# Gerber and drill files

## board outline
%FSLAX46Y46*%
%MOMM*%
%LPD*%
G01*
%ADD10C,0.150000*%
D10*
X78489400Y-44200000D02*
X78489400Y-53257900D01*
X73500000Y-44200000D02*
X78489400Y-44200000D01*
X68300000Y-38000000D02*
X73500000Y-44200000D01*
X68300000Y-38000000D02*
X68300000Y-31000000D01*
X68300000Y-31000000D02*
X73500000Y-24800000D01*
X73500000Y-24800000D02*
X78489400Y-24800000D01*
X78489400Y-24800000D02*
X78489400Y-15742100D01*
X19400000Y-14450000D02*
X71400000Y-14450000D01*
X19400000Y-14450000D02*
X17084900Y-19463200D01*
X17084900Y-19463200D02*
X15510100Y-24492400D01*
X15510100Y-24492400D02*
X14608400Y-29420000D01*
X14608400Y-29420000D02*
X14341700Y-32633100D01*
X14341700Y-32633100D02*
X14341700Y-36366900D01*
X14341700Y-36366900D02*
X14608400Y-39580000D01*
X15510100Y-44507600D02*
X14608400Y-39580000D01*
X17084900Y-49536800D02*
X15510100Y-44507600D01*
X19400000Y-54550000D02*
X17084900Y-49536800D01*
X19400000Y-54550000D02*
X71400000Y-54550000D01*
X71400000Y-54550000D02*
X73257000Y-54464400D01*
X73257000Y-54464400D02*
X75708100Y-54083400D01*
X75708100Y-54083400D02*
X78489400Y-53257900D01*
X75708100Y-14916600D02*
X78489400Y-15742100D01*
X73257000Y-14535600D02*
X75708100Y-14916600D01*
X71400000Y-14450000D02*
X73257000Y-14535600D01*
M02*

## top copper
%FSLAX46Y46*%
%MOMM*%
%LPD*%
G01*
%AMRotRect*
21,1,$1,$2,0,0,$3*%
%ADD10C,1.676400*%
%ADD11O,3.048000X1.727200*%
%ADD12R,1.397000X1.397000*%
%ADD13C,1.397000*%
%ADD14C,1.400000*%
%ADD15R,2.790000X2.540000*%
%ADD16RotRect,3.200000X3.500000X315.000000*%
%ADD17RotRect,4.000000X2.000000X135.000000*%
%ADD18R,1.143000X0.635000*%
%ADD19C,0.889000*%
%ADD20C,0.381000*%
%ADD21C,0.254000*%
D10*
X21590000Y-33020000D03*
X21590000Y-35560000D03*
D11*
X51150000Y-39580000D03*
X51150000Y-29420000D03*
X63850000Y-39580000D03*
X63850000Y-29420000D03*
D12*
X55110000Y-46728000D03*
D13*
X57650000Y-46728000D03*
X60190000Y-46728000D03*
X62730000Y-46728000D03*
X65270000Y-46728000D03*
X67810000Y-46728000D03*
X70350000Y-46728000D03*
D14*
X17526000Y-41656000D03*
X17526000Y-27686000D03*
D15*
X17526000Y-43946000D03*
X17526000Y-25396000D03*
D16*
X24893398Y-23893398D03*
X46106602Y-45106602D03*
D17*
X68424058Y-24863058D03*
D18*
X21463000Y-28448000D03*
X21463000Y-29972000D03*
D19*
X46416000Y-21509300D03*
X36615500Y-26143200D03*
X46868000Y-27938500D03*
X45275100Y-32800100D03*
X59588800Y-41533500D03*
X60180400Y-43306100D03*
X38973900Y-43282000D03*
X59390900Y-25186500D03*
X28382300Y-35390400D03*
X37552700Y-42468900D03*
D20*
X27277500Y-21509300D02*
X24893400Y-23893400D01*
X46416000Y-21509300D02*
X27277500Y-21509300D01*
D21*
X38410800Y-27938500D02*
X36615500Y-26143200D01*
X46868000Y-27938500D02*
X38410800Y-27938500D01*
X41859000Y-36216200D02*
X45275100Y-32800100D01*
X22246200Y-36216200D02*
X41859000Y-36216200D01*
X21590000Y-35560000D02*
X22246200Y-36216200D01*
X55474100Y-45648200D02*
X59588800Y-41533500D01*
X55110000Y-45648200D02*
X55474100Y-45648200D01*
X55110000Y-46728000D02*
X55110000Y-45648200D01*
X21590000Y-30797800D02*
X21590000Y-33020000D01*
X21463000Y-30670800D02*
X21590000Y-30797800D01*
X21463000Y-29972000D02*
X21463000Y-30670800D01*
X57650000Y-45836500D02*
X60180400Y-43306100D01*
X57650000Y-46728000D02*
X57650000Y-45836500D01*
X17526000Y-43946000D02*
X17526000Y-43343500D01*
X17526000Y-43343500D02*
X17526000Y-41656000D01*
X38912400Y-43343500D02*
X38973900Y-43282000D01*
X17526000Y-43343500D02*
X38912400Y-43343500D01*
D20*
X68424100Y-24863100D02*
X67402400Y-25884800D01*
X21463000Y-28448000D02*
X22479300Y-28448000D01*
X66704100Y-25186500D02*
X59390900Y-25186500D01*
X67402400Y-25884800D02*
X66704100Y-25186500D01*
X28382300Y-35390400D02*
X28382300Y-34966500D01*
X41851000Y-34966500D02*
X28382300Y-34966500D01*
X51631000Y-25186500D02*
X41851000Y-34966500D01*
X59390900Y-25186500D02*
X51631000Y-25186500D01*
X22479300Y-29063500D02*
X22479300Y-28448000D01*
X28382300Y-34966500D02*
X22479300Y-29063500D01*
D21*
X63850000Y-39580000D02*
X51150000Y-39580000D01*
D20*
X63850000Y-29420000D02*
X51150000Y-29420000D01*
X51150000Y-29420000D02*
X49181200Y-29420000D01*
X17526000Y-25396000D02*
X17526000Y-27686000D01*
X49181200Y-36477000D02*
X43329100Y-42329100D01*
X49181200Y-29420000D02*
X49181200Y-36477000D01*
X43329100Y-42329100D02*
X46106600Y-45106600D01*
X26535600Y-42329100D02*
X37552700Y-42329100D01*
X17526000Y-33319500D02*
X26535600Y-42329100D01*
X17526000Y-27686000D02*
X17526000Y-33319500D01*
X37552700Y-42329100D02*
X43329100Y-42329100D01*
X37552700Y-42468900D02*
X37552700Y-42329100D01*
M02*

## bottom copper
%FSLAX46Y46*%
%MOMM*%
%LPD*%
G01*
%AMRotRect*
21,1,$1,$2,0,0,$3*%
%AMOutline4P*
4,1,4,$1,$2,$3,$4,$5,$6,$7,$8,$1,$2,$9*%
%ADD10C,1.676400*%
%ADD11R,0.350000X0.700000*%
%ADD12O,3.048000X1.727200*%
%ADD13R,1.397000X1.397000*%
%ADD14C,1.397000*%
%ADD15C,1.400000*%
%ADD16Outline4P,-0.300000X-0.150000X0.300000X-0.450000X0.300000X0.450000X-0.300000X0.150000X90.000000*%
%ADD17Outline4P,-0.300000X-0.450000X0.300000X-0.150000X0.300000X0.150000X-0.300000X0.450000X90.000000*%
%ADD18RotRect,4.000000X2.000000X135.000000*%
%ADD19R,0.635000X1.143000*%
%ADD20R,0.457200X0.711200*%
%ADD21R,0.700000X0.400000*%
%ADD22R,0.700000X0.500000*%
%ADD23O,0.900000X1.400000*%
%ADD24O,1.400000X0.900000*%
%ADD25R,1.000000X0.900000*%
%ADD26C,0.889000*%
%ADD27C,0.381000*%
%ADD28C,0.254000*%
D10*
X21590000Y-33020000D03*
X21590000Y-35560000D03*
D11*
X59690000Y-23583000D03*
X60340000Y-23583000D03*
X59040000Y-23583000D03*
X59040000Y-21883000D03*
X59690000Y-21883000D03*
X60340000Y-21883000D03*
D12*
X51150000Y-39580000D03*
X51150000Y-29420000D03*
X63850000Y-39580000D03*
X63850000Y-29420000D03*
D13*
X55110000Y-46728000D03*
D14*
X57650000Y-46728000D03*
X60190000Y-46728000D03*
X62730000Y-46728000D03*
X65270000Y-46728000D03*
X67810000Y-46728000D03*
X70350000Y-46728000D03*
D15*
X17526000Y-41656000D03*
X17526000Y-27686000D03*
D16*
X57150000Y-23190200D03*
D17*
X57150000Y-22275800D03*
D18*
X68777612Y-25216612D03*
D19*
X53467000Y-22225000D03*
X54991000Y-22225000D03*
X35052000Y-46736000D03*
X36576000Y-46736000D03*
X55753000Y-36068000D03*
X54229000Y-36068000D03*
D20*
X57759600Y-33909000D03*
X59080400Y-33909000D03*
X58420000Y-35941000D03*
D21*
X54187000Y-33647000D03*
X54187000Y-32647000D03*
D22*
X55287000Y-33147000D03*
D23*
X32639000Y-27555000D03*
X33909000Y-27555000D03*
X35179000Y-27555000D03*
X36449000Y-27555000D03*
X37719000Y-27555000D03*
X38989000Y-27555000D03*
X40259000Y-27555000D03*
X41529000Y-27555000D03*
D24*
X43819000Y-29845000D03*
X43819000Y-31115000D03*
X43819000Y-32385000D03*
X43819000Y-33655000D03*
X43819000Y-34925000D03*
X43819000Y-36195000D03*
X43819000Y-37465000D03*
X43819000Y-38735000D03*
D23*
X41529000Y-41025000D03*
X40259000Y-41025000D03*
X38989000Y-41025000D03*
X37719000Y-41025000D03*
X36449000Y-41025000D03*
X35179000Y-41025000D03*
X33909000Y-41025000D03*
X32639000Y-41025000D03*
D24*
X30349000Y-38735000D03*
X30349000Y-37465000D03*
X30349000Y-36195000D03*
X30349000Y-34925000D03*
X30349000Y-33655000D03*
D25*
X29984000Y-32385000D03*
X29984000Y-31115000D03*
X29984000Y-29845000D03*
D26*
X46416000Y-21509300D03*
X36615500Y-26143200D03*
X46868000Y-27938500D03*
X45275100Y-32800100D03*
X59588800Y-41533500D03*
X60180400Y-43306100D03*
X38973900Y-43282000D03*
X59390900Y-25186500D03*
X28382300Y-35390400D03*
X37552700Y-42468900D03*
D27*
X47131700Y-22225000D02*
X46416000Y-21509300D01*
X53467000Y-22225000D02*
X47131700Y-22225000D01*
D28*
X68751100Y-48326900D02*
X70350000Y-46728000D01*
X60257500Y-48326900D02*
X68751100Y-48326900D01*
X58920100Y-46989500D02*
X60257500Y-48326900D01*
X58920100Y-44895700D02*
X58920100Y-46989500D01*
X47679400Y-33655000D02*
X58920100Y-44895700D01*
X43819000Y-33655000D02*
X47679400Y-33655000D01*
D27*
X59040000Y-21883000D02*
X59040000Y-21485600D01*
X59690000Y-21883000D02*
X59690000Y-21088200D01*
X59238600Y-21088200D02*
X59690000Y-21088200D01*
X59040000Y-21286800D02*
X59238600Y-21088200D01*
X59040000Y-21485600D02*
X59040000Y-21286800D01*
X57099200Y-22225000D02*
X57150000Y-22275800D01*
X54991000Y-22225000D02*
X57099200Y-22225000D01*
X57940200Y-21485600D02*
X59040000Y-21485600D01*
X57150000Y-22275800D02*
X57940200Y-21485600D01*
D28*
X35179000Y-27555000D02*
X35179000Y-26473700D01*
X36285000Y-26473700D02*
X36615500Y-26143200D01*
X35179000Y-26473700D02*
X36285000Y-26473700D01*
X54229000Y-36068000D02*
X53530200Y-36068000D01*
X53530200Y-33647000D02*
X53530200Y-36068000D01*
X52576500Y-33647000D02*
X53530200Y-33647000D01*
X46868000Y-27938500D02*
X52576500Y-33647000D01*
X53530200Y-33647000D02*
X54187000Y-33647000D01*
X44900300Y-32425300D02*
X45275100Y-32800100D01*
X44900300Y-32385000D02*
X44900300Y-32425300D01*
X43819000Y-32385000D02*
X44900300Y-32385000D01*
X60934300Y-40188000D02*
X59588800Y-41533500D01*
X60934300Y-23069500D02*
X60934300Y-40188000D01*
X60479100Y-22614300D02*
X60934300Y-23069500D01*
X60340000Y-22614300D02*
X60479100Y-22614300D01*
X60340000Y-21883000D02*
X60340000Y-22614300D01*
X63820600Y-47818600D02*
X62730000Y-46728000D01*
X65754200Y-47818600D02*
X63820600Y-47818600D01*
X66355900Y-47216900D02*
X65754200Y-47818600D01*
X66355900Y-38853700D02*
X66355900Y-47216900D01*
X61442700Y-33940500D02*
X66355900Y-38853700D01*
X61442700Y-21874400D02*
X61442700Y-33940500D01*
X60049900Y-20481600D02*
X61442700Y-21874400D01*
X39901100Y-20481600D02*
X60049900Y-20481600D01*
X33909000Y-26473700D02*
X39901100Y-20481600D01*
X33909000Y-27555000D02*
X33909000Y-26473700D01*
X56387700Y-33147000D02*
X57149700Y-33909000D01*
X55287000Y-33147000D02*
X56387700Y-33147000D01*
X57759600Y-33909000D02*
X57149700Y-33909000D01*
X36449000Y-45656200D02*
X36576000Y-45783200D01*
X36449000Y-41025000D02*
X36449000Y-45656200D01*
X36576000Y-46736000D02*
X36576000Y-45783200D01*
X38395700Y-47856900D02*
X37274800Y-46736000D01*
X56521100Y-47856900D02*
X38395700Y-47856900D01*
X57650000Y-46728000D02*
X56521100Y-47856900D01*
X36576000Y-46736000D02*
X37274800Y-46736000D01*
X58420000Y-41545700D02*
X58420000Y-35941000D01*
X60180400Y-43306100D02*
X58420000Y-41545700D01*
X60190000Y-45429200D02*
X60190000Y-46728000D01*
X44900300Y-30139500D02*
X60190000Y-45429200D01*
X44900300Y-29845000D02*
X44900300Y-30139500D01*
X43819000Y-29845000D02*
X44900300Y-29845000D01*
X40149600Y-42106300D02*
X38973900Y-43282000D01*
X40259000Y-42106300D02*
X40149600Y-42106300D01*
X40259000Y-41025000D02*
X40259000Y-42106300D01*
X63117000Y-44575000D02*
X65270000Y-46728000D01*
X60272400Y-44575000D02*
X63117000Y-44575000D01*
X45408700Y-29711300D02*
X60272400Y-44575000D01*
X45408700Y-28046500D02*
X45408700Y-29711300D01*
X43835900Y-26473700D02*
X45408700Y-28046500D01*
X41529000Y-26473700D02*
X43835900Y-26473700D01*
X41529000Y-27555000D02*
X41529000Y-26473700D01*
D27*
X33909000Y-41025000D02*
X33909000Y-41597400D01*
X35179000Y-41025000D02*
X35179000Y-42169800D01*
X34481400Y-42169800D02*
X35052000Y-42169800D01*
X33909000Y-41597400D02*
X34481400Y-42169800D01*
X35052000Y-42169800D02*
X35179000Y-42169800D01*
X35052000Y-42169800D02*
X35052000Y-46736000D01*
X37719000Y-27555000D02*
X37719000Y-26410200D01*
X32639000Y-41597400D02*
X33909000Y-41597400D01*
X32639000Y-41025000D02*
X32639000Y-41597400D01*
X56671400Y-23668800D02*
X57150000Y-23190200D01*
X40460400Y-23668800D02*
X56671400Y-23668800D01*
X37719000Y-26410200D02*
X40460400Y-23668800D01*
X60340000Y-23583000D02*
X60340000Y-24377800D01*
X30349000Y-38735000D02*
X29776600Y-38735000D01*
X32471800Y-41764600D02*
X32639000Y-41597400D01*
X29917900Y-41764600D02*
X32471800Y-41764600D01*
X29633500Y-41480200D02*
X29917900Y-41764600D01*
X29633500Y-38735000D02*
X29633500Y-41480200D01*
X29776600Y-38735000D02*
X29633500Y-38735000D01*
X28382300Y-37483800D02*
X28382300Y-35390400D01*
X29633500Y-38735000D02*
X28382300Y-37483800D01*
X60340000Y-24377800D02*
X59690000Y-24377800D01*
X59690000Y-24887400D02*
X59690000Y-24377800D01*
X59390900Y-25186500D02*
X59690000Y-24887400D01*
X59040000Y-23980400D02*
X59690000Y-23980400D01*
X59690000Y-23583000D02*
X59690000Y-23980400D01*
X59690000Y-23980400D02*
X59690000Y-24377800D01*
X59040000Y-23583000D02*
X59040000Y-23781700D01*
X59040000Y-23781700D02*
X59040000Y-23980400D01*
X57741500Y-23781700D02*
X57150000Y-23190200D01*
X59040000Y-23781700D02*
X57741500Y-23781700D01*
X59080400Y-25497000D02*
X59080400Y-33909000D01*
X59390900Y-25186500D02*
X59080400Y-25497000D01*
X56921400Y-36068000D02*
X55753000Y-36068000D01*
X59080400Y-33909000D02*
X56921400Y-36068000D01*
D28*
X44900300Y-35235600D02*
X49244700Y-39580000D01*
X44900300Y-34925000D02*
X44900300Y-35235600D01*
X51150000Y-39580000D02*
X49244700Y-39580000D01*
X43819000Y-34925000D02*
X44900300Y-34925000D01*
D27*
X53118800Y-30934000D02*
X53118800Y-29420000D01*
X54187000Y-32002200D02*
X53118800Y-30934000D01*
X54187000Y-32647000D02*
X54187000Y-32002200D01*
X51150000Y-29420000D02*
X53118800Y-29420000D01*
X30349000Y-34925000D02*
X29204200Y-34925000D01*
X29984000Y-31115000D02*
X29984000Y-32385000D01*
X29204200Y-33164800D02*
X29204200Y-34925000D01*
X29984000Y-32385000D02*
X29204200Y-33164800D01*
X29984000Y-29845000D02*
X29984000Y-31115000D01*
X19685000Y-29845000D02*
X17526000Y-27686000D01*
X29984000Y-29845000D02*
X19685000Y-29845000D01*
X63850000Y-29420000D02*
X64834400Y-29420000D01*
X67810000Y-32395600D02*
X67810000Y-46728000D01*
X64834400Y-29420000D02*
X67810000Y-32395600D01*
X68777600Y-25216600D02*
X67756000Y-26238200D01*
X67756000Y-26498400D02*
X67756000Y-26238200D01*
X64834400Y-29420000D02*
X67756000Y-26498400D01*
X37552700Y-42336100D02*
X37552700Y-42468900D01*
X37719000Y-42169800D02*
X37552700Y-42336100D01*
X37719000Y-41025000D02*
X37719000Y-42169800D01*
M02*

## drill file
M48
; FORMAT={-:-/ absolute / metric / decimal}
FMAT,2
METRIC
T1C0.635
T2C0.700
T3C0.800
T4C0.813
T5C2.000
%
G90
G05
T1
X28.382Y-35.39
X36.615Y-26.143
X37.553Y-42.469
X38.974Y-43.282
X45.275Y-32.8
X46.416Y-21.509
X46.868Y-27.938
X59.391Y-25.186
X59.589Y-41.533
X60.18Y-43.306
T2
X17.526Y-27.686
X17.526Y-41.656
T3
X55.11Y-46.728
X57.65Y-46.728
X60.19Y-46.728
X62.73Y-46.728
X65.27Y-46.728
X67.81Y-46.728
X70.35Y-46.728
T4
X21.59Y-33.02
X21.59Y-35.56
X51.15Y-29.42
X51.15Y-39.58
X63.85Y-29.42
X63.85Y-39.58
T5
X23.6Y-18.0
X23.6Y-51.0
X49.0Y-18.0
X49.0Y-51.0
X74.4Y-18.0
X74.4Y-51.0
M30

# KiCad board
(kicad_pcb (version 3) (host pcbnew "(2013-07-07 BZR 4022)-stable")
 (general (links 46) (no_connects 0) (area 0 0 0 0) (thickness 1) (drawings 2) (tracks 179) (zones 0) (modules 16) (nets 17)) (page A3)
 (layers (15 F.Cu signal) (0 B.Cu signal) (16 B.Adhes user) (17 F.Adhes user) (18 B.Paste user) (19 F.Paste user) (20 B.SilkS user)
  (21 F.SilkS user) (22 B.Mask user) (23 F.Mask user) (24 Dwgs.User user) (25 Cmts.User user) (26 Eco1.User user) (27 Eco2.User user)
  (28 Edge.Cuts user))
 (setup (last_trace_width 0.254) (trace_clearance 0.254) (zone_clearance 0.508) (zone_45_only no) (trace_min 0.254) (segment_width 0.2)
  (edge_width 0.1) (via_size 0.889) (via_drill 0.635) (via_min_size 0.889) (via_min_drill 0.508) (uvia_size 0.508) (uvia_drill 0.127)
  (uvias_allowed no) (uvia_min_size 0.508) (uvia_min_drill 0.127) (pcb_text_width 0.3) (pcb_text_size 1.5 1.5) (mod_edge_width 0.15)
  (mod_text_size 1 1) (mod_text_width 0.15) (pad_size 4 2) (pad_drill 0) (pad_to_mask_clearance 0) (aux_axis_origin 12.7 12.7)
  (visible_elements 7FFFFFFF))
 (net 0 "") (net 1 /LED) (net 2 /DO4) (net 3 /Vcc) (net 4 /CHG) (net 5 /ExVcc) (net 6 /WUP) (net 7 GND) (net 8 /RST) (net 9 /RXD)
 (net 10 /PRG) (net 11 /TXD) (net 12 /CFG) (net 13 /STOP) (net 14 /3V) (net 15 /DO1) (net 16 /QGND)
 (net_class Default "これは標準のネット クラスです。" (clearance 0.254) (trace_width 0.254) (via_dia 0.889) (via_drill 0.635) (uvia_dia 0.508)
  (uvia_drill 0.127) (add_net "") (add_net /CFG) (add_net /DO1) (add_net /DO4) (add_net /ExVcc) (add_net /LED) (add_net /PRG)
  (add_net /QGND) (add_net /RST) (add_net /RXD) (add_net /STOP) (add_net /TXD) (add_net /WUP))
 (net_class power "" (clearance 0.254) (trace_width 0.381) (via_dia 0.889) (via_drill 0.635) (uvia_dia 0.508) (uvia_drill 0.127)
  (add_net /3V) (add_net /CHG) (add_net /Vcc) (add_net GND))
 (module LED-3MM (layer F.Cu) (at 21.59 34.29 270)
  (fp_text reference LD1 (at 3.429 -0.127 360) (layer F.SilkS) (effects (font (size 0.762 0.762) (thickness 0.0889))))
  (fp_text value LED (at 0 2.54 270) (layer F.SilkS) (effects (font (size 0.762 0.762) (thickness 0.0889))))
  (pad 1 thru_hole circle (at -1.27 0 270) (size 1.6764 1.6764) (drill 0.8128) (layers *.Cu *.Mask F.SilkS) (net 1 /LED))
  (pad 2 thru_hole circle (at 1.27 0 270) (size 1.6764 1.6764) (drill 0.8128) (layers *.Cu *.Mask F.SilkS) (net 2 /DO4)))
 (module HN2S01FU (layer B.Cu) (at 59.69 22.733 90)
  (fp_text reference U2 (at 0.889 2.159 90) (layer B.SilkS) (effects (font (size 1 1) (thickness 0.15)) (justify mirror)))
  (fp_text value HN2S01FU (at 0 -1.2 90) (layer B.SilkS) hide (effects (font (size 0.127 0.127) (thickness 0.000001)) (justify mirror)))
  (pad 2 smd rect (at -0.85 0 90) (size 0.7 0.35) (layers B.Cu B.Paste B.Mask) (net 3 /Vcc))
  (pad 1 smd rect (at -0.85 0.65 90) (size 0.7 0.35) (layers B.Cu B.Paste B.Mask) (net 3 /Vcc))
  (pad 3 smd rect (at -0.85 -0.65 90) (size 0.7 0.35) (layers B.Cu B.Paste B.Mask) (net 3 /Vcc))
  (pad 4 smd rect (at 0.85 -0.65 90) (size 0.7 0.35) (layers B.Cu B.Paste B.Mask) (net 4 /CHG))
  (pad 5 smd rect (at 0.85 0 90) (size 0.7 0.35) (layers B.Cu B.Paste B.Mask) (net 4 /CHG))
  (pad 6 smd rect (at 0.85 0.65 90) (size 0.7 0.35) (layers B.Cu B.Paste B.Mask) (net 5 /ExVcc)))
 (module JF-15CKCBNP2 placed (layer F.Cu) (at 57.5 34.5 180)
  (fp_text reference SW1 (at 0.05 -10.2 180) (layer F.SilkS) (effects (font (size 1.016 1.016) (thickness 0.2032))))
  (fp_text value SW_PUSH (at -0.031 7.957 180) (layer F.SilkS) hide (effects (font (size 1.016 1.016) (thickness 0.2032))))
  (pad 1 thru_hole oval (at 6.35 -5.08 180) (size 3.048 1.7272) (drill 0.8128) (layers *.Cu *.Mask F.SilkS) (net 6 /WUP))
  (pad 2 thru_hole oval (at 6.35 5.08 180) (size 3.048 1.7272) (drill 0.8128) (layers *.Cu *.Mask F.SilkS) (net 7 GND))
  (pad 1 thru_hole oval (at -6.35 -5.08 180) (size 3.048 1.7272) (drill 0.8128) (layers *.Cu *.Mask F.SilkS) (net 6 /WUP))
  (pad 2 thru_hole oval (at -6.35 5.08 180) (size 3.048 1.7272) (drill 0.8128) (layers *.Cu *.Mask F.SilkS) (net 7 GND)))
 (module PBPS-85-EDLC (layer F.Cu) (at 49 34.5)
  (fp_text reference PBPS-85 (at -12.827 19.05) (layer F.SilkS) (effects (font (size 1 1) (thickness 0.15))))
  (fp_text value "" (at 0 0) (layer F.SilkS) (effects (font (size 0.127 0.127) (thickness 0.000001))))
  (fp_line (start 29.4894 9.7) (end 29.4894 18.7579) (layer Edge.Cuts) (width 0.15))
  (fp_line (start 24.5 9.7) (end 29.4894 9.7) (layer Edge.Cuts) (width 0.15))
  (fp_line (start 19.3 3.5) (end 24.5 9.7) (layer Edge.Cuts) (width 0.15))
  (fp_line (start 19.3 3.5) (end 19.3 -3.5) (layer Edge.Cuts) (width 0.15))
  (fp_line (start 19.3 -3.5) (end 24.5 -9.7) (layer Edge.Cuts) (width 0.15))
  (fp_line (start 24.5 -9.7) (end 29.4894 -9.7) (layer Edge.Cuts) (width 0.15))
  (fp_line (start 29.4894 -9.7) (end 29.4894 -18.7579) (layer Edge.Cuts) (width 0.15))
  (fp_line (start -29.6 -20.05) (end 22.4 -20.05) (layer Edge.Cuts) (width 0.15))
  (fp_line (start -29.6 -20.05) (end -31.9151 -15.0368) (layer Edge.Cuts) (width 0.15))
  (fp_line (start -31.9151 -15.0368) (end -33.4899 -10.0076) (layer Edge.Cuts) (width 0.15))
  (fp_line (start -33.4899 -10.0076) (end -34.3916 -5.08) (layer Edge.Cuts) (width 0.15))
  (fp_line (start -34.3916 -5.08) (end -34.6583 -1.8669) (layer Edge.Cuts) (width 0.15))
  (fp_line (start -34.6583 -1.8669) (end -34.6583 1.8669) (layer Edge.Cuts) (width 0.15))
  (fp_line (start -34.6583 1.8669) (end -34.3916 5.08) (layer Edge.Cuts) (width 0.15))
  (fp_line (start -33.4899 10.0076) (end -34.3916 5.08) (layer Edge.Cuts) (width 0.15))
  (fp_line (start -31.9151 15.0368) (end -33.4899 10.0076) (layer Edge.Cuts) (width 0.15))
  (fp_line (start -29.6 20.05) (end -31.9151 15.0368) (layer Edge.Cuts) (width 0.15))
  (fp_line (start -29.6 20.05) (end 22.4 20.05) (layer Edge.Cuts) (width 0.15))
  (fp_line (start 22.4 20.05) (end 24.257 19.9644) (layer Edge.Cuts) (width 0.15))
  (fp_line (start 24.257 19.9644) (end 26.7081 19.5834) (layer Edge.Cuts) (width 0.15))
  (fp_line (start 26.7081 19.5834) (end 29.4894 18.7579) (layer Edge.Cuts) (width 0.15))
  (fp_line (start 26.7081 -19.5834) (end 29.4894 -18.7579) (layer Edge.Cuts) (width 0.15))
  (fp_line (start 24.257 -19.9644) (end 26.7081 -19.5834) (layer Edge.Cuts) (width 0.15))
  (fp_line (start 22.4 -20.05) (end 24.257 -19.9644) (layer Edge.Cuts) (width 0.15))
  (pad "" np_thru_hole circle (at 0 -16.5) (size 2 2) (drill 2) (layers *.Cu *.Mask F.SilkS) (clearance 1))
  (pad "" np_thru_hole circle (at 0 16.5) (size 2 2) (drill 2) (layers *.Cu *.Mask F.SilkS) (clearance 1))
  (pad "" np_thru_hole circle (at -25.4 -16.5) (size 2 2) (drill 2) (layers *.Cu *.Mask F.SilkS) (clearance 1))
  (pad "" np_thru_hole circle (at -25.4 16.5) (size 2 2) (drill 2) (layers *.Cu *.Mask F.SilkS) (clearance 1))
  (pad "" np_thru_hole circle (at 25.4 -16.5) (size 2 2) (drill 2) (layers *.Cu *.Mask F.SilkS) (clearance 1))
  (pad "" np_thru_hole circle (at 25.4 16.5) (size 2 2) (drill 2) (layers *.Cu *.Mask F.SilkS) (clearance 1)))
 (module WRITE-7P (layer F.Cu) (at 62.73 46.728)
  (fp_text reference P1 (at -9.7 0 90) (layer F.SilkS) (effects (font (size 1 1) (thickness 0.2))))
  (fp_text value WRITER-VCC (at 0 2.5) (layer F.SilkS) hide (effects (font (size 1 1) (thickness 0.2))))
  (pad 0 thru_hole rect (at -7.62 0) (size 1.397 1.397) (drill 0.8) (layers *.Cu *.Mask F.SilkS) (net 5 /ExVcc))
  (pad 1 thru_hole circle (at -5.08 0) (size 1.397 1.397) (drill 0.8) (layers *.Cu *.SilkS *.Mask) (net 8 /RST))
  (pad 2 thru_hole circle (at -2.54 0) (size 1.397 1.397) (drill 0.8) (layers *.Cu *.SilkS *.Mask) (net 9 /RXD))
  (pad 3 thru_hole circle (at 0 0) (size 1.397 1.397) (drill 0.8) (layers *.Cu *.SilkS *.Mask) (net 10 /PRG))
  (pad 4 thru_hole circle (at 2.54 0) (size 1.397 1.397) (drill 0.8) (layers *.Cu *.SilkS *.Mask) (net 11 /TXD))
  (pad 5 thru_hole circle (at 5.08 0) (size 1.397 1.397) (drill 0.8) (layers *.Cu *.SilkS *.Mask) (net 7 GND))
  (pad 6 thru_hole circle (at 7.62 0) (size 1.397 1.397) (drill 0.8) (layers *.Cu *.SilkS *.Mask) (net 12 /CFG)))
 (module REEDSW (layer F.Cu) (at 17.526 34.671 90)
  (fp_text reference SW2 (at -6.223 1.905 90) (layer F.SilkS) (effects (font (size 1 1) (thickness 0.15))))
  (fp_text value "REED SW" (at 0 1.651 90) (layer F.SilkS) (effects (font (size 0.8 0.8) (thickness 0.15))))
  (pad 1 thru_hole circle (at -6.985 0 90) (size 1.4 1.4) (drill 0.7) (layers *.Cu *.Mask F.SilkS) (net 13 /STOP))
  (pad 2 thru_hole circle (at 6.985 0 90) (size 1.4 1.4) (drill 0.7) (layers *.Cu *.Mask F.SilkS) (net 7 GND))
  (pad 1 smd rect (at -9.275 0 90) (size 2.54 2.79) (layers F.Cu F.Paste F.Mask) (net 13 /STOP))
  (pad 2 smd rect (at 9.275 0 90) (size 2.54 2.79) (layers F.Cu F.Paste F.Mask) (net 7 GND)))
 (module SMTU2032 (layer F.Cu) (at 35.5 34.5 315)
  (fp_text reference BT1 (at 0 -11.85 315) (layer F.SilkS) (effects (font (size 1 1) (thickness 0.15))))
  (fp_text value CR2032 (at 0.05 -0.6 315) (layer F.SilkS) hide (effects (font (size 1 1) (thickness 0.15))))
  (pad 1 smd rect (at -15 0 315) (size 3.2 3.5) (layers F.Cu F.Paste F.Mask) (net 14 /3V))
  (pad 2 smd rect (at 15 0 315) (size 3.2 3.5) (layers F.Cu F.Paste F.Mask) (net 7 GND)))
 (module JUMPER (layer B.Cu) (at 57.15 22.733 90)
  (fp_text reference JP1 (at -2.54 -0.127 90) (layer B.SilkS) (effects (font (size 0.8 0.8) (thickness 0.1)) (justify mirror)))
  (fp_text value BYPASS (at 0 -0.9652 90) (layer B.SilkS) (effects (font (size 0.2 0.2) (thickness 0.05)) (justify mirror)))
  (pad 1 smd trapezoid (at -0.4572 0 90) (size 0.6 0.6) (rect_delta -0.3 0) (layers B.Cu B.Paste B.Mask) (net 3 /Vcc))
  (pad 2 smd trapezoid (at 0.4572 0 90) (size 0.6 0.6) (rect_delta 0.3 0) (layers B.Cu B.Paste B.Mask) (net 4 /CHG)))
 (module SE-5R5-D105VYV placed (layer F.Cu) (at 77.97 34.409 135)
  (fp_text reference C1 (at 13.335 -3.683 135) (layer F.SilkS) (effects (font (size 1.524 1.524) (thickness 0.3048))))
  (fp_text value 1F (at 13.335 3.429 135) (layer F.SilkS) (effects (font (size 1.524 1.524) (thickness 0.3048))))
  (pad 1 smd rect (at 13.5 0 135) (size 4 2) (layers F.Cu F.Paste F.Mask) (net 3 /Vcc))
  (pad 2 smd rect (at 13 0 135) (size 4 2) (layers B.Cu B.Paste B.Mask) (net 7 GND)))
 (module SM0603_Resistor (layer F.Cu) (at 21.463 29.21 270)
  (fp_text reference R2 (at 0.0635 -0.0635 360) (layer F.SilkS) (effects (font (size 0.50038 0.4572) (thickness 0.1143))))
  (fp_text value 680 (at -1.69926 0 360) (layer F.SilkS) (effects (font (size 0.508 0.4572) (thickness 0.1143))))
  (pad 1 smd rect (at -0.762 0 270) (size 0.635 1.143) (layers F.Cu F.Paste F.Mask) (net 3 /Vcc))
  (pad 2 smd rect (at 0.762 0 270) (size 0.635 1.143) (layers F.Cu F.Paste F.Mask) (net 1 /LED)))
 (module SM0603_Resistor (layer B.Cu) (at 54.229 22.225)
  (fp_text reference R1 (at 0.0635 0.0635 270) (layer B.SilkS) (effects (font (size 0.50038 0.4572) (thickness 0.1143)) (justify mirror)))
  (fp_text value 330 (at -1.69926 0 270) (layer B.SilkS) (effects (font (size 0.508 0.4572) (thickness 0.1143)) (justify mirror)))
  (pad 1 smd rect (at -0.762 0) (size 0.635 1.143) (layers B.Cu B.Paste B.Mask) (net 14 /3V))
  (pad 2 smd rect (at 0.762 0) (size 0.635 1.143) (layers B.Cu B.Paste B.Mask) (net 4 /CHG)))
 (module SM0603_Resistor (layer B.Cu) (at 35.814 46.736)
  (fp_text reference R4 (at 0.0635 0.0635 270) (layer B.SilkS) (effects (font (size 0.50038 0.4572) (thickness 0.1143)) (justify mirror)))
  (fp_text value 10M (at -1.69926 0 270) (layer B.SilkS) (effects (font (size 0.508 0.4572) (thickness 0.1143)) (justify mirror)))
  (pad 1 smd rect (at -0.762 0) (size 0.635 1.143) (layers B.Cu B.Paste B.Mask) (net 3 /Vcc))
  (pad 2 smd rect (at 0.762 0) (size 0.635 1.143) (layers B.Cu B.Paste B.Mask) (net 8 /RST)))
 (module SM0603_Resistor (layer B.Cu) (at 54.991 36.068 180)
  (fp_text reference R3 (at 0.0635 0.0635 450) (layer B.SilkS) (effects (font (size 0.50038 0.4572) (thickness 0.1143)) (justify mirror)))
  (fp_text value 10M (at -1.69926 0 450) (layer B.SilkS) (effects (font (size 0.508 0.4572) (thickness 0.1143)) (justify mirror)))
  (pad 1 smd rect (at -0.762 0 180) (size 0.635 1.143) (layers B.Cu B.Paste B.Mask) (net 3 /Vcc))
  (pad 2 smd rect (at 0.762 0 180) (size 0.635 1.143) (layers B.Cu B.Paste B.Mask) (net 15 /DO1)))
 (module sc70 (layer B.Cu) (at 58.42 34.925)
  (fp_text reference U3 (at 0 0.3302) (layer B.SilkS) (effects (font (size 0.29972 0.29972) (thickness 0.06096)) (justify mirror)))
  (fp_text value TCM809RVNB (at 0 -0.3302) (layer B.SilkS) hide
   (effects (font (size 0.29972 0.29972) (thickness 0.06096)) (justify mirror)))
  (pad 1 smd rect (at -0.6604 -1.016) (size 0.4572 0.7112) (layers B.Cu B.Paste B.Mask) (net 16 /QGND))
  (pad 3 smd rect (at 0.6604 -1.016) (size 0.4572 0.7112) (layers B.Cu B.Paste B.Mask) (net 3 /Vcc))
  (pad 2 smd rect (at 0 1.016) (size 0.4572 0.7112) (layers B.Cu B.Paste B.Mask) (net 8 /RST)))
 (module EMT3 (layer B.Cu) (at 54.737 33.147 90)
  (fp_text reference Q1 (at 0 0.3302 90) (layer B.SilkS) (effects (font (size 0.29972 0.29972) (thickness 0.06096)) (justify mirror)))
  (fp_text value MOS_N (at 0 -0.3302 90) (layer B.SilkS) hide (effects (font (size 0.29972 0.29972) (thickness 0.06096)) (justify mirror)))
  (pad G smd rect (at -0.5 -0.55 90) (size 0.4 0.7) (layers B.Cu B.Paste B.Mask) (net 15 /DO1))
  (pad S smd rect (at 0.5 -0.55 90) (size 0.4 0.7) (layers B.Cu B.Paste B.Mask) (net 7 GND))
  (pad D smd rect (at 0 0.55 90) (size 0.5 0.7) (layers B.Cu B.Paste B.Mask) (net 16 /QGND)))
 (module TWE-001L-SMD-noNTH (layer B.Cu) (at 37.084 34.29 270)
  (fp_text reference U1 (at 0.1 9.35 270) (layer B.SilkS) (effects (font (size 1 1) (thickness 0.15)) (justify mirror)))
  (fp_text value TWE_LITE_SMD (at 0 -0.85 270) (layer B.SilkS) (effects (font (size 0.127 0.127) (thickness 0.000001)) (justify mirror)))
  (pad 1 smd oval (at -6.735 4.445 180) (size 0.9 1.4) (layers B.Cu B.Paste B.Mask))
  (pad 2 smd oval (at -6.735 3.175 180) (size 0.9 1.4) (layers B.Cu B.Paste B.Mask) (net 10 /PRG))
  (pad 3 smd oval (at -6.735 1.905 180) (size 0.9 1.4) (layers B.Cu B.Paste B.Mask) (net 15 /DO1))
  (pad 4 smd oval (at -6.735 0.635 180) (size 0.9 1.4) (layers B.Cu B.Paste B.Mask))
  (pad 5 smd oval (at -6.735 -0.635 180) (size 0.9 1.4) (layers B.Cu B.Paste B.Mask) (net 3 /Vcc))
  (pad 6 smd oval (at -6.735 -1.905 180) (size 0.9 1.4) (layers B.Cu B.Paste B.Mask))
  (pad 7 smd oval (at -6.735 -3.175 180) (size 0.9 1.4) (layers B.Cu B.Paste B.Mask))
  (pad 8 smd oval (at -6.735 -4.445 180) (size 0.9 1.4) (layers B.Cu B.Paste B.Mask) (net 11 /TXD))
  (pad 9 smd oval (at -4.445 -6.735 270) (size 0.9 1.4) (layers B.Cu B.Paste B.Mask) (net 9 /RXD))
  (pad 10 smd oval (at -3.175 -6.735 270) (size 0.9 1.4) (layers B.Cu B.Paste B.Mask))
  (pad 11 smd oval (at -1.905 -6.735 270) (size 0.9 1.4) (layers B.Cu B.Paste B.Mask) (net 2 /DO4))
  (pad 12 smd oval (at -0.635 -6.735 270) (size 0.9 1.4) (layers B.Cu B.Paste B.Mask) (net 12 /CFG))
  (pad 13 smd oval (at 0.635 -6.735 270) (size 0.9 1.4) (layers B.Cu B.Paste B.Mask) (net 6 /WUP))
  (pad 14 smd oval (at 1.905 -6.735 270) (size 0.9 1.4) (layers B.Cu B.Paste B.Mask))
  (pad 15 smd oval (at 3.175 -6.735 270) (size 0.9 1.4) (layers B.Cu B.Paste B.Mask))
  (pad 16 smd oval (at 4.445 -6.735 270) (size 0.9 1.4) (layers B.Cu B.Paste B.Mask))
  (pad 17 smd oval (at 6.735 -4.445 180) (size 0.9 1.4) (layers B.Cu B.Paste B.Mask))
  (pad 18 smd oval (at 6.735 -3.175 180) (size 0.9 1.4) (layers B.Cu B.Paste B.Mask) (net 13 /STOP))
  (pad 19 smd oval (at 6.735 -1.905 180) (size 0.9 1.4) (layers B.Cu B.Paste B.Mask))
  (pad 20 smd oval (at 6.735 -0.635 180) (size 0.9 1.4) (layers B.Cu B.Paste B.Mask) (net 7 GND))
  (pad 21 smd oval (at 6.735 0.635 180) (size 0.9 1.4) (layers B.Cu B.Paste B.Mask) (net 8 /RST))
  (pad 22 smd oval (at 6.735 1.905 180) (size 0.9 1.4) (layers B.Cu B.Paste B.Mask) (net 3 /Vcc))
  (pad 23 smd oval (at 6.735 3.175 180) (size 0.9 1.4) (layers B.Cu B.Paste B.Mask) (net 3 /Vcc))
  (pad 24 smd oval (at 6.735 4.445 180) (size 0.9 1.4) (layers B.Cu B.Paste B.Mask) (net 3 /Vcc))
  (pad 25 smd oval (at 4.445 6.735 270) (size 0.9 1.4) (layers B.Cu B.Paste B.Mask) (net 3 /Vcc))
  (pad 26 smd oval (at 3.175 6.735 270) (size 0.9 1.4) (layers B.Cu B.Paste B.Mask))
  (pad 27 smd oval (at 1.905 6.735 270) (size 0.9 1.4) (layers B.Cu B.Paste B.Mask))
  (pad 28 smd oval (at 0.635 6.735 270) (size 0.9 1.4) (layers B.Cu B.Paste B.Mask) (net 7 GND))
  (pad 29 smd oval (at -0.635 6.735 270) (size 0.9 1.4) (layers B.Cu B.Paste B.Mask))
  (pad 30 smd rect (at -1.905 7.1 270) (size 0.9 1) (layers B.Cu B.Paste B.Mask) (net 7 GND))
  (pad 31 smd rect (at -3.175 7.1 270) (size 0.9 1) (layers B.Cu B.Paste B.Mask) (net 7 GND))
  (pad 32 smd rect (at -4.445 7.1 270) (size 0.9 1) (layers B.Cu B.Paste B.Mask) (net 7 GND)))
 (via (at 46.416 21.5093) (size 0.889) (layers F.Cu B.Cu) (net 14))
 (segment (start 47.1317 22.225) (end 46.416 21.5093) (width 0.381) (layer B.Cu) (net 14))
 (segment (start 53.467 22.225) (end 47.1317 22.225) (width 0.381) (layer B.Cu) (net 14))
 (segment (start 27.2775 21.5093) (end 24.8934 23.8934) (width 0.381) (layer F.Cu) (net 14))
 (segment (start 46.416 21.5093) (end 27.2775 21.5093) (width 0.381) (layer F.Cu) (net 14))
 (segment (start 68.7511 48.3269) (end 70.35 46.728) (width 0.254) (layer B.Cu) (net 12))
 (segment (start 60.2575 48.3269) (end 68.7511 48.3269) (width 0.254) (layer B.Cu) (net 12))
 (segment (start 58.9201 46.9895) (end 60.2575 48.3269) (width 0.254) (layer B.Cu) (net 12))
 (segment (start 58.9201 44.8957) (end 58.9201 46.9895) (width 0.254) (layer B.Cu) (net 12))
 (segment (start 47.6794 33.655) (end 58.9201 44.8957) (width 0.254) (layer B.Cu) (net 12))
 (segment (start 43.819 33.655) (end 47.6794 33.655) (width 0.254) (layer B.Cu) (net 12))
 (segment (start 59.04 21.883) (end 59.04 21.4856) (width 0.381) (layer B.Cu) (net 4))
 (segment (start 59.69 21.883) (end 59.69 21.0882) (width 0.381) (layer B.Cu) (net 4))
 (segment (start 59.2386 21.0882) (end 59.69 21.0882) (width 0.381) (layer B.Cu) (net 4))
 (segment (start 59.04 21.2868) (end 59.2386 21.0882) (width 0.381) (layer B.Cu) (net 4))
 (segment (start 59.04 21.4856) (end 59.04 21.2868) (width 0.381) (layer B.Cu) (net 4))
 (segment (start 57.0992 22.225) (end 57.15 22.2758) (width 0.381) (layer B.Cu) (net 4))
 (segment (start 54.991 22.225) (end 57.0992 22.225) (width 0.381) (layer B.Cu) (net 4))
 (segment (start 57.9402 21.4856) (end 59.04 21.4856) (width 0.381) (layer B.Cu) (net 4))
 (segment (start 57.15 22.2758) (end 57.9402 21.4856) (width 0.381) (layer B.Cu) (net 4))
 (via (at 36.6155 26.1432) (size 0.889) (layers F.Cu B.Cu) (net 15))
 (via (at 46.868 27.9385) (size 0.889) (layers F.Cu B.Cu) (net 15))
 (segment (start 35.179 27.555) (end 35.179 26.4737) (width 0.254) (layer B.Cu) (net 15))
 (segment (start 36.285 26.4737) (end 36.6155 26.1432) (width 0.254) (layer B.Cu) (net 15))
 (segment (start 35.179 26.4737) (end 36.285 26.4737) (width 0.254) (layer B.Cu) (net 15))
 (segment (start 38.4108 27.9385) (end 36.6155 26.1432) (width 0.254) (layer F.Cu) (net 15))
 (segment (start 46.868 27.9385) (end 38.4108 27.9385) (width 0.254) (layer F.Cu) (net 15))
 (segment (start 54.229 36.068) (end 53.5302 36.068) (width 0.254) (layer B.Cu) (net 15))
 (segment (start 53.5302 33.647) (end 53.5302 36.068) (width 0.254) (layer B.Cu) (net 15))
 (segment (start 52.5765 33.647) (end 53.5302 33.647) (width 0.254) (layer B.Cu) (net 15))
 (segment (start 46.868 27.9385) (end 52.5765 33.647) (width 0.254) (layer B.Cu) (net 15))
 (segment (start 53.5302 33.647) (end 54.187 33.647) (width 0.254) (layer B.Cu) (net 15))
 (via (at 45.2751 32.8001) (size 0.889) (layers F.Cu B.Cu) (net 2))
 (segment (start 44.9003 32.4253) (end 45.2751 32.8001) (width 0.254) (layer B.Cu) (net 2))
 (segment (start 44.9003 32.385) (end 44.9003 32.4253) (width 0.254) (layer B.Cu) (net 2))
 (segment (start 43.819 32.385) (end 44.9003 32.385) (width 0.254) (layer B.Cu) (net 2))
 (segment (start 41.859 36.2162) (end 45.2751 32.8001) (width 0.254) (layer F.Cu) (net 2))
 (segment (start 22.2462 36.2162) (end 41.859 36.2162) (width 0.254) (layer F.Cu) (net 2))
 (segment (start 21.59 35.56) (end 22.2462 36.2162) (width 0.254) (layer F.Cu) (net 2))
 (via (at 59.5888 41.5335) (size 0.889) (layers F.Cu B.Cu) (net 5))
 (segment (start 60.9343 40.188) (end 59.5888 41.5335) (width 0.254) (layer B.Cu) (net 5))
 (segment (start 60.9343 23.0695) (end 60.9343 40.188) (width 0.254) (layer B.Cu) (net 5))
 (segment (start 60.4791 22.6143) (end 60.9343 23.0695) (width 0.254) (layer B.Cu) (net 5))
 (segment (start 60.34 22.6143) (end 60.4791 22.6143) (width 0.254) (layer B.Cu) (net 5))
 (segment (start 55.4741 45.6482) (end 59.5888 41.5335) (width 0.254) (layer F.Cu) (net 5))
 (segment (start 55.11 45.6482) (end 55.4741 45.6482) (width 0.254) (layer F.Cu) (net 5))
 (segment (start 60.34 21.883) (end 60.34 22.6143) (width 0.254) (layer B.Cu) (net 5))
 (segment (start 55.11 46.728) (end 55.11 45.6482) (width 0.254) (layer F.Cu) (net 5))
 (segment (start 21.59 30.7978) (end 21.59 33.02) (width 0.254) (layer F.Cu) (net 1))
 (segment (start 21.463 30.6708) (end 21.59 30.7978) (width 0.254) (layer F.Cu) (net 1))
 (segment (start 21.463 29.972) (end 21.463 30.6708) (width 0.254) (layer F.Cu) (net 1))
 (segment (start 63.8206 47.8186) (end 62.73 46.728) (width 0.254) (layer B.Cu) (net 10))
 (segment (start 65.7542 47.8186) (end 63.8206 47.8186) (width 0.254) (layer B.Cu) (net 10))
 (segment (start 66.3559 47.2169) (end 65.7542 47.8186) (width 0.254) (layer B.Cu) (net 10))
 (segment (start 66.3559 38.8537) (end 66.3559 47.2169) (width 0.254) (layer B.Cu) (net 10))
 (segment (start 61.4427 33.9405) (end 66.3559 38.8537) (width 0.254) (layer B.Cu) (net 10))
 (segment (start 61.4427 21.8744) (end 61.4427 33.9405) (width 0.254) (layer B.Cu) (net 10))
 (segment (start 60.0499 20.4816) (end 61.4427 21.8744) (width 0.254) (layer B.Cu) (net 10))
 (segment (start 39.9011 20.4816) (end 60.0499 20.4816) (width 0.254) (layer B.Cu) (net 10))
 (segment (start 33.909 26.4737) (end 39.9011 20.4816) (width 0.254) (layer B.Cu) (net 10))
 (segment (start 33.909 27.555) (end 33.909 26.4737) (width 0.254) (layer B.Cu) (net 10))
 (segment (start 56.3877 33.147) (end 57.1497 33.909) (width 0.254) (layer B.Cu) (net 16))
 (segment (start 55.287 33.147) (end 56.3877 33.147) (width 0.254) (layer B.Cu) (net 16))
 (segment (start 57.7596 33.909) (end 57.1497 33.909) (width 0.254) (layer B.Cu) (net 16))
 (via (at 60.1804 43.3061) (size 0.889) (layers F.Cu B.Cu) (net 8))
 (segment (start 36.449 45.6562) (end 36.576 45.7832) (width 0.254) (layer B.Cu) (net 8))
 (segment (start 36.449 41.025) (end 36.449 45.6562) (width 0.254) (layer B.Cu) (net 8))
 (segment (start 36.576 46.736) (end 36.576 45.7832) (width 0.254) (layer B.Cu) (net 8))
 (segment (start 38.3957 47.8569) (end 37.2748 46.736) (width 0.254) (layer B.Cu) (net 8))
 (segment (start 56.5211 47.8569) (end 38.3957 47.8569) (width 0.254) (layer B.Cu) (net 8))
 (segment (start 57.65 46.728) (end 56.5211 47.8569) (width 0.254) (layer B.Cu) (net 8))
 (segment (start 36.576 46.736) (end 37.2748 46.736) (width 0.254) (layer B.Cu) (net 8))
 (segment (start 58.42 41.5457) (end 58.42 35.941) (width 0.254) (layer B.Cu) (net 8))
 (segment (start 60.1804 43.3061) (end 58.42 41.5457) (width 0.254) (layer B.Cu) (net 8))
 (segment (start 57.65 45.8365) (end 60.1804 43.3061) (width 0.254) (layer F.Cu) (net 8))
 (segment (start 57.65 46.728) (end 57.65 45.8365) (width 0.254) (layer F.Cu) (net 8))
 (segment (start 60.19 45.4292) (end 60.19 46.728) (width 0.254) (layer B.Cu) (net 9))
 (segment (start 44.9003 30.1395) (end 60.19 45.4292) (width 0.254) (layer B.Cu) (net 9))
 (segment (start 44.9003 29.845) (end 44.9003 30.1395) (width 0.254) (layer B.Cu) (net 9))
 (segment (start 43.819 29.845) (end 44.9003 29.845) (width 0.254) (layer B.Cu) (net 9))
 (via (at 38.9739 43.282) (size 0.889) (layers F.Cu B.Cu) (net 13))
 (segment (start 40.1496 42.1063) (end 38.9739 43.282) (width 0.254) (layer B.Cu) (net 13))
 (segment (start 40.259 42.1063) (end 40.1496 42.1063) (width 0.254) (layer B.Cu) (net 13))
 (segment (start 40.259 41.025) (end 40.259 42.1063) (width 0.254) (layer B.Cu) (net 13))
 (segment (start 17.526 43.946) (end 17.526 43.3435) (width 0.254) (layer F.Cu) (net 13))
 (segment (start 17.526 43.3435) (end 17.526 41.656) (width 0.254) (layer F.Cu) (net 13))
 (segment (start 38.9124 43.3435) (end 38.9739 43.282) (width 0.254) (layer F.Cu) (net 13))
 (segment (start 17.526 43.3435) (end 38.9124 43.3435) (width 0.254) (layer F.Cu) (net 13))
 (segment (start 63.117 44.575) (end 65.27 46.728) (width 0.254) (layer B.Cu) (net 11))
 (segment (start 60.2724 44.575) (end 63.117 44.575) (width 0.254) (layer B.Cu) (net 11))
 (segment (start 45.4087 29.7113) (end 60.2724 44.575) (width 0.254) (layer B.Cu) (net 11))
 (segment (start 45.4087 28.0465) (end 45.4087 29.7113) (width 0.254) (layer B.Cu) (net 11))
 (segment (start 43.8359 26.4737) (end 45.4087 28.0465) (width 0.254) (layer B.Cu) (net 11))
 (segment (start 41.529 26.4737) (end 43.8359 26.4737) (width 0.254) (layer B.Cu) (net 11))
 (segment (start 41.529 27.555) (end 41.529 26.4737) (width 0.254) (layer B.Cu) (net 11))
 (via (at 59.3909 25.1865) (size 0.889) (layers F.Cu B.Cu) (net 3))
 (via (at 28.3823 35.3904) (size 0.889) (layers F.Cu B.Cu) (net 3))
 (segment (start 33.909 41.025) (end 33.909 41.5974) (width 0.381) (layer B.Cu) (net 3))
 (segment (start 35.179 41.025) (end 35.179 42.1698) (width 0.381) (layer B.Cu) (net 3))
 (segment (start 34.4814 42.1698) (end 35.052 42.1698) (width 0.381) (layer B.Cu) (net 3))
 (segment (start 33.909 41.5974) (end 34.4814 42.1698) (width 0.381) (layer B.Cu) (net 3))
 (segment (start 35.052 42.1698) (end 35.179 42.1698) (width 0.381) (layer B.Cu) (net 3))
 (segment (start 68.4241 24.8631) (end 67.4024 25.8848) (width 0.381) (layer F.Cu) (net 3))
 (segment (start 35.052 42.1698) (end 35.052 46.736) (width 0.381) (layer B.Cu) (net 3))
 (segment (start 37.719 27.555) (end 37.719 26.4102) (width 0.381) (layer B.Cu) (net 3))
 (segment (start 32.639 41.5974) (end 33.909 41.5974) (width 0.381) (layer B.Cu) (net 3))
 (segment (start 32.639 41.025) (end 32.639 41.5974) (width 0.381) (layer B.Cu) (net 3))
 (segment (start 56.6714 23.6688) (end 57.15 23.1902) (width 0.381) (layer B.Cu) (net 3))
 (segment (start 40.4604 23.6688) (end 56.6714 23.6688) (width 0.381) (layer B.Cu) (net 3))
 (segment (start 37.719 26.4102) (end 40.4604 23.6688) (width 0.381) (layer B.Cu) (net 3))
 (segment (start 60.34 23.583) (end 60.34 24.3778) (width 0.381) (layer B.Cu) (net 3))
 (segment (start 21.463 28.448) (end 22.4793 28.448) (width 0.381) (layer F.Cu) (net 3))
 (segment (start 66.7041 25.1865) (end 59.3909 25.1865) (width 0.381) (layer F.Cu) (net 3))
 (segment (start 67.4024 25.8848) (end 66.7041 25.1865) (width 0.381) (layer F.Cu) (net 3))
 (segment (start 30.349 38.735) (end 29.7766 38.735) (width 0.381) (layer B.Cu) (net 3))
 (segment (start 28.3823 35.3904) (end 28.3823 34.9665) (width 0.381) (layer F.Cu) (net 3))
 (segment (start 41.851 34.9665) (end 28.3823 34.9665) (width 0.381) (layer F.Cu) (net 3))
 (segment (start 51.631 25.1865) (end 41.851 34.9665) (width 0.381) (layer F.Cu) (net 3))
 (segment (start 59.3909 25.1865) (end 51.631 25.1865) (width 0.381) (layer F.Cu) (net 3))
 (segment (start 22.4793 29.0635) (end 22.4793 28.448) (width 0.381) (layer F.Cu) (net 3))
 (segment (start 28.3823 34.9665) (end 22.4793 29.0635) (width 0.381) (layer F.Cu) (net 3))
 (segment (start 32.4718 41.7646) (end 32.639 41.5974) (width 0.381) (layer B.Cu) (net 3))
 (segment (start 29.9179 41.7646) (end 32.4718 41.7646) (width 0.381) (layer B.Cu) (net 3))
 (segment (start 29.6335 41.4802) (end 29.9179 41.7646) (width 0.381) (layer B.Cu) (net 3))
 (segment (start 29.6335 38.735) (end 29.6335 41.4802) (width 0.381) (layer B.Cu) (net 3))
 (segment (start 29.7766 38.735) (end 29.6335 38.735) (width 0.381) (layer B.Cu) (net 3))
 (segment (start 28.3823 37.4838) (end 28.3823 35.3904) (width 0.381) (layer B.Cu) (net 3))
 (segment (start 29.6335 38.735) (end 28.3823 37.4838) (width 0.381) (layer B.Cu) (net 3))
 (segment (start 60.34 24.3778) (end 59.69 24.3778) (width 0.381) (layer B.Cu) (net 3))
 (segment (start 59.69 24.8874) (end 59.69 24.3778) (width 0.381) (layer B.Cu) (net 3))
 (segment (start 59.3909 25.1865) (end 59.69 24.8874) (width 0.381) (layer B.Cu) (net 3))
 (segment (start 59.04 23.9804) (end 59.69 23.9804) (width 0.381) (layer B.Cu) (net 3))
 (segment (start 59.69 23.583) (end 59.69 23.9804) (width 0.381) (layer B.Cu) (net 3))
 (segment (start 59.69 23.9804) (end 59.69 24.3778) (width 0.381) (layer B.Cu) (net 3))
 (segment (start 59.04 23.583) (end 59.04 23.7817) (width 0.381) (layer B.Cu) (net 3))
 (segment (start 59.04 23.7817) (end 59.04 23.9804) (width 0.381) (layer B.Cu) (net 3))
 (segment (start 57.7415 23.7817) (end 57.15 23.1902) (width 0.381) (layer B.Cu) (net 3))
 (segment (start 59.04 23.7817) (end 57.7415 23.7817) (width 0.381) (layer B.Cu) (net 3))
 (segment (start 59.0804 25.497) (end 59.0804 33.909) (width 0.381) (layer B.Cu) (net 3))
 (segment (start 59.3909 25.1865) (end 59.0804 25.497) (width 0.381) (layer B.Cu) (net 3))
 (segment (start 56.9214 36.068) (end 55.753 36.068) (width 0.381) (layer B.Cu) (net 3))
 (segment (start 59.0804 33.909) (end 56.9214 36.068) (width 0.381) (layer B.Cu) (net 3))
 (segment (start 44.9003 35.2356) (end 49.2447 39.58) (width 0.254) (layer B.Cu) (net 6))
 (segment (start 44.9003 34.925) (end 44.9003 35.2356) (width 0.254) (layer B.Cu) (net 6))
 (segment (start 51.15 39.58) (end 49.2447 39.58) (width 0.254) (layer B.Cu) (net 6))
 (segment (start 43.819 34.925) (end 44.9003 34.925) (width 0.254) (layer B.Cu) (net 6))
 (segment (start 63.85 39.58) (end 51.15 39.58) (width 0.254) (layer F.Cu) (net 6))
 (via (at 37.5527 42.4689) (size 0.889) (layers F.Cu B.Cu) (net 7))
 (segment (start 53.1188 30.934) (end 53.1188 29.42) (width 0.381) (layer B.Cu) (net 7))
 (segment (start 54.187 32.0022) (end 53.1188 30.934) (width 0.381) (layer B.Cu) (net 7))
 (segment (start 54.187 32.647) (end 54.187 32.0022) (width 0.381) (layer B.Cu) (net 7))
 (segment (start 51.15 29.42) (end 53.1188 29.42) (width 0.381) (layer B.Cu) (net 7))
 (segment (start 63.85 29.42) (end 51.15 29.42) (width 0.381) (layer F.Cu) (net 7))
 (segment (start 30.349 34.925) (end 29.2042 34.925) (width 0.381) (layer B.Cu) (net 7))
 (segment (start 29.984 31.115) (end 29.984 32.385) (width 0.381) (layer B.Cu) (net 7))
 (segment (start 29.2042 33.1648) (end 29.2042 34.925) (width 0.381) (layer B.Cu) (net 7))
 (segment (start 29.984 32.385) (end 29.2042 33.1648) (width 0.381) (layer B.Cu) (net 7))
 (segment (start 29.984 29.845) (end 29.984 31.115) (width 0.381) (layer B.Cu) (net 7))
 (segment (start 19.685 29.845) (end 17.526 27.686) (width 0.381) (layer B.Cu) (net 7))
 (segment (start 29.984 29.845) (end 19.685 29.845) (width 0.381) (layer B.Cu) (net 7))
 (segment (start 51.15 29.42) (end 49.1812 29.42) (width 0.381) (layer F.Cu) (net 7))
 (segment (start 63.85 29.42) (end 64.8344 29.42) (width 0.381) (layer B.Cu) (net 7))
 (segment (start 67.81 32.3956) (end 67.81 46.728) (width 0.381) (layer B.Cu) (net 7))
 (segment (start 64.8344 29.42) (end 67.81 32.3956) (width 0.381) (layer B.Cu) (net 7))
 (segment (start 68.7776 25.2166) (end 67.756 26.2382) (width 0.381) (layer B.Cu) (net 7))
 (segment (start 67.756 26.4984) (end 67.756 26.2382) (width 0.381) (layer B.Cu) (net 7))
 (segment (start 64.8344 29.42) (end 67.756 26.4984) (width 0.381) (layer B.Cu) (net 7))
 (segment (start 17.526 25.396) (end 17.526 27.686) (width 0.381) (layer F.Cu) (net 7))
 (segment (start 49.1812 36.477) (end 43.3291 42.3291) (width 0.381) (layer F.Cu) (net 7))
 (segment (start 49.1812 29.42) (end 49.1812 36.477) (width 0.381) (layer F.Cu) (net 7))
 (segment (start 43.3291 42.3291) (end 46.1066 45.1066) (width 0.381) (layer F.Cu) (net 7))
 (segment (start 26.5356 42.3291) (end 37.5527 42.3291) (width 0.381) (layer F.Cu) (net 7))
 (segment (start 17.526 33.3195) (end 26.5356 42.3291) (width 0.381) (layer F.Cu) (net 7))
 (segment (start 17.526 27.686) (end 17.526 33.3195) (width 0.381) (layer F.Cu) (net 7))
 (segment (start 37.5527 42.3291) (end 43.3291 42.3291) (width 0.381) (layer F.Cu) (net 7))
 (segment (start 37.5527 42.3361) (end 37.5527 42.4689) (width 0.381) (layer B.Cu) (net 7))
 (segment (start 37.719 42.1698) (end 37.5527 42.3361) (width 0.381) (layer B.Cu) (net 7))
 (segment (start 37.5527 42.4689) (end 37.5527 42.3291) (width 0.381) (layer F.Cu) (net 7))
 (segment (start 37.719 41.025) (end 37.719 42.1698) (width 0.381) (layer B.Cu) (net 7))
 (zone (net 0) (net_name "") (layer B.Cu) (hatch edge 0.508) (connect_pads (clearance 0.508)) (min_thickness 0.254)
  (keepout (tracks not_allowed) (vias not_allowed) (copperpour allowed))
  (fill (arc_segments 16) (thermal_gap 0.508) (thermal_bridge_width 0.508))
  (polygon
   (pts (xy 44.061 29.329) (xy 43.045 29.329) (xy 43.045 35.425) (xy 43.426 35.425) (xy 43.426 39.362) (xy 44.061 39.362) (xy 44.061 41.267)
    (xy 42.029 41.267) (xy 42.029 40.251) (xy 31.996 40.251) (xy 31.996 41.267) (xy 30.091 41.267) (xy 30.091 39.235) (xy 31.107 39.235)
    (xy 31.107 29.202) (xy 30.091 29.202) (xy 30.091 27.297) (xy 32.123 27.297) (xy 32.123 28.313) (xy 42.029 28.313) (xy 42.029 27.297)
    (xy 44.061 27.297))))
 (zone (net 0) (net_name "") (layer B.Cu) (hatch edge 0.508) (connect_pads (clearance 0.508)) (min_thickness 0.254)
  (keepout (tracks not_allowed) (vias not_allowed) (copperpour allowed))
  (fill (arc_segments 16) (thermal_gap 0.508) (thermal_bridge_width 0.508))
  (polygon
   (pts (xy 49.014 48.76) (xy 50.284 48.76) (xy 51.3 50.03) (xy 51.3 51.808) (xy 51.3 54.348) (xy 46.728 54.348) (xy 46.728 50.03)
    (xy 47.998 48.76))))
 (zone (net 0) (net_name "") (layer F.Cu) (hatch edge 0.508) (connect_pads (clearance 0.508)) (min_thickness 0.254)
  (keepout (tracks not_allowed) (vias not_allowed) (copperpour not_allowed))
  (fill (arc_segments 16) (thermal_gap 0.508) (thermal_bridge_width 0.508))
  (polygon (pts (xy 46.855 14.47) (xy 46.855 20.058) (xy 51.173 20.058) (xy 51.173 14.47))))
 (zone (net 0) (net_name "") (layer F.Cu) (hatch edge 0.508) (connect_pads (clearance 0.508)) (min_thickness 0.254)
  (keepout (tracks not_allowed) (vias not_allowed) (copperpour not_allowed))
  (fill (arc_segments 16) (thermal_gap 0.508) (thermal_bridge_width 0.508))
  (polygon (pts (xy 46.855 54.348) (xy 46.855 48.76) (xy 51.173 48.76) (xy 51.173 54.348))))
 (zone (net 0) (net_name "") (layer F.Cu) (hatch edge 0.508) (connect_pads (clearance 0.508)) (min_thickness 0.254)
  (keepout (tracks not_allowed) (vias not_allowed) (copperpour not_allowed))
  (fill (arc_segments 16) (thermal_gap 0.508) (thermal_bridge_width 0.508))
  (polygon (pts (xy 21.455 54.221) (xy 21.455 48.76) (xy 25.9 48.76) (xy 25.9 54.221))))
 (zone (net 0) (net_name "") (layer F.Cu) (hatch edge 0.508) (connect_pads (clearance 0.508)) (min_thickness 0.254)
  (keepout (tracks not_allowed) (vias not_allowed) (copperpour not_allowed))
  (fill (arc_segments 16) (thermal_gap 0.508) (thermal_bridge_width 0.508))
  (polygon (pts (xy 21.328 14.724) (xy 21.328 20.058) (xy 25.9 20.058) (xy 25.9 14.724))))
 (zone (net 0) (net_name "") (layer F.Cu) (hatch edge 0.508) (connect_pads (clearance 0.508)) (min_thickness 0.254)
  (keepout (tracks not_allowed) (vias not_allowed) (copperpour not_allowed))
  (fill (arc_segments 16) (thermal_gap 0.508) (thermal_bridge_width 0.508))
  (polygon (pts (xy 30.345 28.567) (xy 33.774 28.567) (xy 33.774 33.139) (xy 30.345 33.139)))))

